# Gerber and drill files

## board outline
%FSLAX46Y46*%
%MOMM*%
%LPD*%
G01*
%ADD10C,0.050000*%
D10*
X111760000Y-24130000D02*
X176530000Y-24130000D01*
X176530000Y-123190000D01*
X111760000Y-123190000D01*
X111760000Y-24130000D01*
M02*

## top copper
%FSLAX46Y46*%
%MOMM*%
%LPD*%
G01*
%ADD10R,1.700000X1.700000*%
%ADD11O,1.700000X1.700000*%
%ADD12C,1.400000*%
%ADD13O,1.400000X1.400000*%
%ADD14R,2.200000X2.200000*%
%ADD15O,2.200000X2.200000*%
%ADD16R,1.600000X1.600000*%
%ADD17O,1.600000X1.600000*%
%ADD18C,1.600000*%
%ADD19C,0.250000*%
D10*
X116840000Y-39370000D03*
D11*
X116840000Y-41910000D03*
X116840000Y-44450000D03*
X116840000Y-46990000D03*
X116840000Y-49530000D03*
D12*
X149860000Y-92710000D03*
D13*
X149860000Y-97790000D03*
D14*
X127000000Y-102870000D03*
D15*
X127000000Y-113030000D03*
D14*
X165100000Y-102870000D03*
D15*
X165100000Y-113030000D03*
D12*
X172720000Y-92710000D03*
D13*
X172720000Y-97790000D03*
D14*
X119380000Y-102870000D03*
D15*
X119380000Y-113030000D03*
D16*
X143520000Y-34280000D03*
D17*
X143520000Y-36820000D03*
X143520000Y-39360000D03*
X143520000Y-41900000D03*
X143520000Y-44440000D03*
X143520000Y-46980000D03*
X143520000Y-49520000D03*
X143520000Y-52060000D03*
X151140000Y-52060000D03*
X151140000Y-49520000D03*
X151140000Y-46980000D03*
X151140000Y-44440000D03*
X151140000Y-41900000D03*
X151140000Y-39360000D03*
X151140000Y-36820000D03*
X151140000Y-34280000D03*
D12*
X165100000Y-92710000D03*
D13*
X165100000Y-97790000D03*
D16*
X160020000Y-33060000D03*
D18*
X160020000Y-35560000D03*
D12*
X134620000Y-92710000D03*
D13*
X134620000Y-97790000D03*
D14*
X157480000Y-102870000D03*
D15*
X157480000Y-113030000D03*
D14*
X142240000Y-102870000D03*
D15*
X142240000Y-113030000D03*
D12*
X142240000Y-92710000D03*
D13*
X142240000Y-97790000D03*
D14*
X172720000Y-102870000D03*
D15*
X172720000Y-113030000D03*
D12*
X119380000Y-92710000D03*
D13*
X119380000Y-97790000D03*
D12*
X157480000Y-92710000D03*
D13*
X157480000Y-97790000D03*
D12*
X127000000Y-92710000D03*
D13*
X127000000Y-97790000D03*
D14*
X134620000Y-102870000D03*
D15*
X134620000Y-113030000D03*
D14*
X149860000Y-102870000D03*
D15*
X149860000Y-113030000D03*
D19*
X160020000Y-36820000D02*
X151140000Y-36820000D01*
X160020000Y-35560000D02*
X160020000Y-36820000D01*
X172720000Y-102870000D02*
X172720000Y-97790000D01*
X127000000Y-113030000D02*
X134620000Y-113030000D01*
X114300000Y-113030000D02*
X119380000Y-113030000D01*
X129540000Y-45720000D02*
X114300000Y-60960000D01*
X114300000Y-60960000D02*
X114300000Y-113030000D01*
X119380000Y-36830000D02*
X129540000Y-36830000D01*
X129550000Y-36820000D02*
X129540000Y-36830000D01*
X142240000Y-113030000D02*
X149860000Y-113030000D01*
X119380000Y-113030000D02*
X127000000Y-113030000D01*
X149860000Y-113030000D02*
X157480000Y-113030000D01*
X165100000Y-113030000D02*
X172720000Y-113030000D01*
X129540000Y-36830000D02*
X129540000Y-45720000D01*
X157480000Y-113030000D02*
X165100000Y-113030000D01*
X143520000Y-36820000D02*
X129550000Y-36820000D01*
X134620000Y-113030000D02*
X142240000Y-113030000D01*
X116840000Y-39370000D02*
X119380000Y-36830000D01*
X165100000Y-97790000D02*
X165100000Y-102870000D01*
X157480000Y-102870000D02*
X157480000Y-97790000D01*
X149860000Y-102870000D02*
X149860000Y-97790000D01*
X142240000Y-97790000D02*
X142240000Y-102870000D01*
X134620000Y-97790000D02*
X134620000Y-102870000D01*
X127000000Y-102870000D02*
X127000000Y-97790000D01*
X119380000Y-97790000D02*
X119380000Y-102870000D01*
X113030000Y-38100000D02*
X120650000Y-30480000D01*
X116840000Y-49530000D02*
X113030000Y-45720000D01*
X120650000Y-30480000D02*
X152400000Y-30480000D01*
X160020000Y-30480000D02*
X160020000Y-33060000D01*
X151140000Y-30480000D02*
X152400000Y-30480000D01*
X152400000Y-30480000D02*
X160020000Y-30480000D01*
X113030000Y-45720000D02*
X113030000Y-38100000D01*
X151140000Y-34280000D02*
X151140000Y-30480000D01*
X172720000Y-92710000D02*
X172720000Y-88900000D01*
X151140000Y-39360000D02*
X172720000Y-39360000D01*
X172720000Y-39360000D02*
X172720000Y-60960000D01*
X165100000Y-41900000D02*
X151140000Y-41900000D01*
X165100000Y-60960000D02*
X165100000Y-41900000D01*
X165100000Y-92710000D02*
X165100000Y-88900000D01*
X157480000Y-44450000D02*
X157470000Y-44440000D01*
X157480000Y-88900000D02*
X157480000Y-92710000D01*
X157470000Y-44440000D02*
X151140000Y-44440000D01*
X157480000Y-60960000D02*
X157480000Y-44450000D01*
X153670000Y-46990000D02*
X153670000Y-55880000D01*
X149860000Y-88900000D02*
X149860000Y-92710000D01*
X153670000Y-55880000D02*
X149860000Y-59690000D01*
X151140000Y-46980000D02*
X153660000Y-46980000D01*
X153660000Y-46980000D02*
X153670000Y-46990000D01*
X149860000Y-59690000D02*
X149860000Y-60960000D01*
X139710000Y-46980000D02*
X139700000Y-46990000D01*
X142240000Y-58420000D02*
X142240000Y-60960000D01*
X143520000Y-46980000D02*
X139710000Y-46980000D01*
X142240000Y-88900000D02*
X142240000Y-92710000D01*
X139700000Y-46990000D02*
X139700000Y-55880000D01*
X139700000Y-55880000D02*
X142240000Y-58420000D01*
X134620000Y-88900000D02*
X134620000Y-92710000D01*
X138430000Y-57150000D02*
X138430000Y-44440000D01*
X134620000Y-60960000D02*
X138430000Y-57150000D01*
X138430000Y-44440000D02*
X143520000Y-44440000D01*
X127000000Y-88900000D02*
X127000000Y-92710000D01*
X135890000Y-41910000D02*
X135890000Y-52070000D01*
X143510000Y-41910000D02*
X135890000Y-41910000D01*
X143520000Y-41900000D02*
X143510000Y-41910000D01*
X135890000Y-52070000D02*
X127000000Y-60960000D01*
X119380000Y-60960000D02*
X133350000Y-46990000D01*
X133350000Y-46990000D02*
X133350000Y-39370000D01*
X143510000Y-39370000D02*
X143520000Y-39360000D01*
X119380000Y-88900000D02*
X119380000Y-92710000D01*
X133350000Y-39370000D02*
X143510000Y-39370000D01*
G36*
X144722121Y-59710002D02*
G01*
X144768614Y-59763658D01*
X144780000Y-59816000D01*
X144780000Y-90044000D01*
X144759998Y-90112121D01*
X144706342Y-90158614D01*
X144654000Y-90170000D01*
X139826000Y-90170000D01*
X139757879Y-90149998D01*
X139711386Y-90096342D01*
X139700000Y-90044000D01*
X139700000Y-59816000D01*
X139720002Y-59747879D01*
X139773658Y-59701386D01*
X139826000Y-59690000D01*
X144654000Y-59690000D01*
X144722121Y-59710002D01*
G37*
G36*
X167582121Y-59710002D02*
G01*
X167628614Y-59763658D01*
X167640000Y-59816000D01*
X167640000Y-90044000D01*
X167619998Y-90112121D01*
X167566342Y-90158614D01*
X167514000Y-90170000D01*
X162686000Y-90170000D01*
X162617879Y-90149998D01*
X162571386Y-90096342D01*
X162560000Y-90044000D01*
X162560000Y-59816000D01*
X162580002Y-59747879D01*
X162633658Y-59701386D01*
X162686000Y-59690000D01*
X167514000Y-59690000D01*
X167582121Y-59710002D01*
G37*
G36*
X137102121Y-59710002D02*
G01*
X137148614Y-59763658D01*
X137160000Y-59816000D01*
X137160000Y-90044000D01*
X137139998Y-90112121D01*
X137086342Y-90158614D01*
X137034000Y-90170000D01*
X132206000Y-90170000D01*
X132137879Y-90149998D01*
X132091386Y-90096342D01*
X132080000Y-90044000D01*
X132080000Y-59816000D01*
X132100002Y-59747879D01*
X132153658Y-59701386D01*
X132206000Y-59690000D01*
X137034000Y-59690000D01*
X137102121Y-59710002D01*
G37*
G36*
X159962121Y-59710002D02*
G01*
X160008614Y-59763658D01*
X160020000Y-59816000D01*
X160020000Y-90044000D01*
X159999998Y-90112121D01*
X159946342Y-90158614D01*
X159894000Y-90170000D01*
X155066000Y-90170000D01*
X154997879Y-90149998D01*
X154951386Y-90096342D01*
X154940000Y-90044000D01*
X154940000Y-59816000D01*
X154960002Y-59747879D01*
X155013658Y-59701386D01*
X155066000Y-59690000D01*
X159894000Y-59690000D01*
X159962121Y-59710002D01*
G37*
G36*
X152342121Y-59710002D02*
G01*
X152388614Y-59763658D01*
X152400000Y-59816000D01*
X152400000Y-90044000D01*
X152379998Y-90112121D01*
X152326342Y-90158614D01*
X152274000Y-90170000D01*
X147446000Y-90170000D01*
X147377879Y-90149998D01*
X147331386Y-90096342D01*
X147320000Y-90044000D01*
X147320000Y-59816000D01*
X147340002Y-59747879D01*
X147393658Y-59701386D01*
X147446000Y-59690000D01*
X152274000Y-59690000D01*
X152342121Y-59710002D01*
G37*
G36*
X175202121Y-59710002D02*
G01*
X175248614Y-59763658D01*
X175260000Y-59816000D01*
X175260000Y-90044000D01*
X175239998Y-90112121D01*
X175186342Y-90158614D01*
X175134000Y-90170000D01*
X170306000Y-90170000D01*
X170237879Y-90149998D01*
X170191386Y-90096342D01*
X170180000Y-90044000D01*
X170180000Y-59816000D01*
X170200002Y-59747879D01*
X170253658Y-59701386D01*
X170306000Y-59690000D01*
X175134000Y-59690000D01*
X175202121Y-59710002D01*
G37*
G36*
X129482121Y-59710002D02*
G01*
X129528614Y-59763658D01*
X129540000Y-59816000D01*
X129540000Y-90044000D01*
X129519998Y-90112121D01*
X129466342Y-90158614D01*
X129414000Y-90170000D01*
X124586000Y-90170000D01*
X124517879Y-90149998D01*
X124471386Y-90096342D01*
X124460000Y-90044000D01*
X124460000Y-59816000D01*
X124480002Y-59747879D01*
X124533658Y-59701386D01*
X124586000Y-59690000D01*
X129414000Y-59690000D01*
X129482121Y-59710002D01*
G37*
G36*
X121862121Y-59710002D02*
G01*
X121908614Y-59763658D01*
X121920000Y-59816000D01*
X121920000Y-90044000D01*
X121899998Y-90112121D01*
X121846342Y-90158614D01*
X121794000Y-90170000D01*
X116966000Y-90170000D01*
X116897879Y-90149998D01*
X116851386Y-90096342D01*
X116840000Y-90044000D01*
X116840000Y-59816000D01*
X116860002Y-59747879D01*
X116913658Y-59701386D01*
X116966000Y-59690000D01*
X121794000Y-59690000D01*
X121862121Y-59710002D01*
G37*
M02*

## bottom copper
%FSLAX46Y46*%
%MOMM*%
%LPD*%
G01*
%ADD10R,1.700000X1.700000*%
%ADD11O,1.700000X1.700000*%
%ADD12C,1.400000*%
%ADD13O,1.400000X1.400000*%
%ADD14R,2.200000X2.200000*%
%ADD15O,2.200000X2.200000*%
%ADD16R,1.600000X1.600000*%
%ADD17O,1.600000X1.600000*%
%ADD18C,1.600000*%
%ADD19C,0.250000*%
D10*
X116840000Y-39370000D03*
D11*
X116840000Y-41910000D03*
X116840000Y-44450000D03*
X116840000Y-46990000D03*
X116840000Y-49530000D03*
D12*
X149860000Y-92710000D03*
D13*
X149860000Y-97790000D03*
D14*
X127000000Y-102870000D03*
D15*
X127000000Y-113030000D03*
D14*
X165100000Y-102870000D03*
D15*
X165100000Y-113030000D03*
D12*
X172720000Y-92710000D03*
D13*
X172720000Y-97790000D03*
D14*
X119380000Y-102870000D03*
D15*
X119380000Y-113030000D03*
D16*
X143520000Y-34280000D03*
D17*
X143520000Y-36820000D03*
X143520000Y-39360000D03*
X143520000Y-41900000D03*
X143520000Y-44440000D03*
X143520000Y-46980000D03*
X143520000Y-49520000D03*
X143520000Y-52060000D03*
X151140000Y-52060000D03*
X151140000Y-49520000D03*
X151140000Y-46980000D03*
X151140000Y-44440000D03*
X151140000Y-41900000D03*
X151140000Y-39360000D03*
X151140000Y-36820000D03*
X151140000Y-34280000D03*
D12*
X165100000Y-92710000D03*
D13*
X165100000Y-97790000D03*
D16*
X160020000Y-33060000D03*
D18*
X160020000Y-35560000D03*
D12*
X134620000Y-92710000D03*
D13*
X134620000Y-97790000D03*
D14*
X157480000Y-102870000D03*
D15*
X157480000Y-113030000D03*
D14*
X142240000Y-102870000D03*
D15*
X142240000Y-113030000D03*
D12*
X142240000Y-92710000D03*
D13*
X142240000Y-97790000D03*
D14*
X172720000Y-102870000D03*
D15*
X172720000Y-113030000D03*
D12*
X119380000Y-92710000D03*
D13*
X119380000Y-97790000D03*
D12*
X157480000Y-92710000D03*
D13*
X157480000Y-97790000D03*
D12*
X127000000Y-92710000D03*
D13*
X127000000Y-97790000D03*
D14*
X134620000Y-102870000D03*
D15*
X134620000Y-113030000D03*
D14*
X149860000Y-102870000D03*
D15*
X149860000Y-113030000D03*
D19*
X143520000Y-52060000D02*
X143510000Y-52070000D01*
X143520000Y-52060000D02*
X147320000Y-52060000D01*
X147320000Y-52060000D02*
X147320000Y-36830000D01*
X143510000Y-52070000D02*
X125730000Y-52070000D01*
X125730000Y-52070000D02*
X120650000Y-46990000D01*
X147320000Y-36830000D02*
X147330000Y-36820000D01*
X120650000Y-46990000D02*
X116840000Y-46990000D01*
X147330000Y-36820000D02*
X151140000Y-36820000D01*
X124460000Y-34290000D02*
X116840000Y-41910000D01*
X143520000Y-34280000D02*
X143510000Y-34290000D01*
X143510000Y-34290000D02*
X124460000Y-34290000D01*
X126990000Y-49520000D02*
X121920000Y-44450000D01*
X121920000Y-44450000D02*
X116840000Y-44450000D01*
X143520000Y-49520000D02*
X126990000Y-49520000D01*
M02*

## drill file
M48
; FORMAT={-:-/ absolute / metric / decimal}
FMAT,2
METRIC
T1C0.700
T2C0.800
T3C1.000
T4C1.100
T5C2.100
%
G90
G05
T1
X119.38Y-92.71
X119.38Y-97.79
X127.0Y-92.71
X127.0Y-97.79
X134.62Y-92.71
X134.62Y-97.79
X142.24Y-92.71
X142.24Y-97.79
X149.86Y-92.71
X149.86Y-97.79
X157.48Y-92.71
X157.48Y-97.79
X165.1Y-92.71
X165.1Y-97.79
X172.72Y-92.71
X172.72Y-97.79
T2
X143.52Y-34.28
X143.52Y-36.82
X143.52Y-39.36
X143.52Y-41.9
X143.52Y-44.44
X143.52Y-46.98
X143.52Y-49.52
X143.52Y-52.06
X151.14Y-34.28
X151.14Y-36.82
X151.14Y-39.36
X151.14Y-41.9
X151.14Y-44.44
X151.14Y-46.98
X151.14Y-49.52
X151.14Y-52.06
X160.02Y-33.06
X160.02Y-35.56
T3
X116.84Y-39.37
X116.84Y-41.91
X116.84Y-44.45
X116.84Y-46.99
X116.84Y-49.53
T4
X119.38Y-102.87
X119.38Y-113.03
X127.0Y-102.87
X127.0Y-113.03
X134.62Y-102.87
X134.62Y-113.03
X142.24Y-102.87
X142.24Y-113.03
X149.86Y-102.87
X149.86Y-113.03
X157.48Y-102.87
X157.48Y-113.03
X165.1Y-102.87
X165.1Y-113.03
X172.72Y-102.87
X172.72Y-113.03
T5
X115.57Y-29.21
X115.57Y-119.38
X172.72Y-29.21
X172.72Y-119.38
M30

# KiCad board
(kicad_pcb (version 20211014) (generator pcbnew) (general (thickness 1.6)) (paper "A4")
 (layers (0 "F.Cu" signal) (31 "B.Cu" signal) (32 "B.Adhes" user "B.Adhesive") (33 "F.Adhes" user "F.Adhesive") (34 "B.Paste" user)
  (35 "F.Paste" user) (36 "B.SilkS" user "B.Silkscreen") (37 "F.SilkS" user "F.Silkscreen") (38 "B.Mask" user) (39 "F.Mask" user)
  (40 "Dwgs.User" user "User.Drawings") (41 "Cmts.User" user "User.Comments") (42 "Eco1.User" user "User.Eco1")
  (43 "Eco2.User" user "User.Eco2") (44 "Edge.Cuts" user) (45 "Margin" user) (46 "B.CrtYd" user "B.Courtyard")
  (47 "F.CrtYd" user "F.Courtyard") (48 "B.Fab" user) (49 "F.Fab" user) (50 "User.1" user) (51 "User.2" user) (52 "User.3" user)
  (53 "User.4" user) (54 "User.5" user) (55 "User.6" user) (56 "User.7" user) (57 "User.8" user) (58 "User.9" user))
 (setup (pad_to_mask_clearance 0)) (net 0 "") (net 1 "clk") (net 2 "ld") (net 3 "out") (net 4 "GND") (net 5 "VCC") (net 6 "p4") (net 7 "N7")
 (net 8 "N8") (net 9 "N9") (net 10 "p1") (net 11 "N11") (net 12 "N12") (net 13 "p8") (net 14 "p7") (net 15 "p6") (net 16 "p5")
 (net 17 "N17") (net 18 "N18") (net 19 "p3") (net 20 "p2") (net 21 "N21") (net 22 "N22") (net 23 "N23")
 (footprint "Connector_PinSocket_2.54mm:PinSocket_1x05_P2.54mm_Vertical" (layer "F.Cu") (at 116.84 39.37)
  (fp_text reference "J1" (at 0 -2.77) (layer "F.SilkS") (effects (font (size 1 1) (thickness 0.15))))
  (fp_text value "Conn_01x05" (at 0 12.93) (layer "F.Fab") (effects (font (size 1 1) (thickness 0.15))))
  (pad "1" thru_hole rect (at 0 0) (size 1.7 1.7) (drill 1) (layers *.Cu *.Mask) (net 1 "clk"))
  (pad "2" thru_hole oval (at 0 2.54) (size 1.7 1.7) (drill 1) (layers *.Cu *.Mask) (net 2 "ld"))
  (pad "3" thru_hole oval (at 0 5.08) (size 1.7 1.7) (drill 1) (layers *.Cu *.Mask) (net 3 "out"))
  (pad "4" thru_hole oval (at 0 7.62) (size 1.7 1.7) (drill 1) (layers *.Cu *.Mask) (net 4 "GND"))
  (pad "5" thru_hole oval (at 0 10.16) (size 1.7 1.7) (drill 1) (layers *.Cu *.Mask) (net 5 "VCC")))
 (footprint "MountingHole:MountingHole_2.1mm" (layer "F.Cu") (at 172.72 29.21)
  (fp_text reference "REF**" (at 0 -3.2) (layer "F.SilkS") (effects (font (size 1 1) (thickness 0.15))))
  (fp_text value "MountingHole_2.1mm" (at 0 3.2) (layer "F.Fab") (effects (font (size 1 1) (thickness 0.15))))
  (pad "" np_thru_hole circle (at 0 0) (size 2.1 2.1) (drill 2.1) (layers *.Cu *.Mask)))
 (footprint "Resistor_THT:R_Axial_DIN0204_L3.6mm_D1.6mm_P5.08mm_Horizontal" (layer "F.Cu") (at 149.86 92.71 -90)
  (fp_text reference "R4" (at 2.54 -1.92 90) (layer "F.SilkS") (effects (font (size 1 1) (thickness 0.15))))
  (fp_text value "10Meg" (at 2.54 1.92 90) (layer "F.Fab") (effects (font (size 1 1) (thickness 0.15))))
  (pad "1" thru_hole circle (at 0 0 270) (size 1.4 1.4) (drill 0.7) (layers *.Cu *.Mask) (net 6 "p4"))
  (pad "2" thru_hole oval (at 5.08 0 270) (size 1.4 1.4) (drill 0.7) (layers *.Cu *.Mask) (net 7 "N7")))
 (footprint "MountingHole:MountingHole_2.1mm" (layer "F.Cu") (at 115.57 119.38)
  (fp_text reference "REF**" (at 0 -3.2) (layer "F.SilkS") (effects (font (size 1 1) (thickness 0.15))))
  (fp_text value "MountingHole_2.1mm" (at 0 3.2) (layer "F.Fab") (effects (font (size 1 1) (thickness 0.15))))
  (pad "" np_thru_hole circle (at 0 0) (size 2.1 2.1) (drill 2.1) (layers *.Cu *.Mask)))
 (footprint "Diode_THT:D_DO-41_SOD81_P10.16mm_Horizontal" (layer "F.Cu") (at 127 102.87 -90)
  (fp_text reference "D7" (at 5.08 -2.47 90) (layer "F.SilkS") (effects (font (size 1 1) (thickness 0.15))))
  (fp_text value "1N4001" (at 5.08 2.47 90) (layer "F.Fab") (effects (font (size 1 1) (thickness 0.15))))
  (pad "1" thru_hole rect (at 0 0 270) (size 2.2 2.2) (drill 1.1) (layers *.Cu *.Mask) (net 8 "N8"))
  (pad "2" thru_hole oval (at 10.16 0 270) (size 2.2 2.2) (drill 1.1) (layers *.Cu *.Mask) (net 1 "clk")))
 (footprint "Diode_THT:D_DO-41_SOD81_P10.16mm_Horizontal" (layer "F.Cu") (at 165.1 102.87 -90)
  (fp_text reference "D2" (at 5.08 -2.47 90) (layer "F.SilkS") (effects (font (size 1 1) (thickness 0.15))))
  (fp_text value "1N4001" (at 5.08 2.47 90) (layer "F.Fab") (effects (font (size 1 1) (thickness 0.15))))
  (pad "1" thru_hole rect (at 0 0 270) (size 2.2 2.2) (drill 1.1) (layers *.Cu *.Mask) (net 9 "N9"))
  (pad "2" thru_hole oval (at 10.16 0 270) (size 2.2 2.2) (drill 1.1) (layers *.Cu *.Mask) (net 1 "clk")))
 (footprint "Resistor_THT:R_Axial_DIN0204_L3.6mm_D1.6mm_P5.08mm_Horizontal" (layer "F.Cu") (at 172.72 92.71 -90)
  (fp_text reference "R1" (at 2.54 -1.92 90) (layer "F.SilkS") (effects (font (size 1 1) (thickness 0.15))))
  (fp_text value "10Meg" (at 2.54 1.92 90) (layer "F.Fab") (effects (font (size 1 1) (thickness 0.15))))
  (pad "1" thru_hole circle (at 0 0 270) (size 1.4 1.4) (drill 0.7) (layers *.Cu *.Mask) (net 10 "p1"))
  (pad "2" thru_hole oval (at 5.08 0 270) (size 1.4 1.4) (drill 0.7) (layers *.Cu *.Mask) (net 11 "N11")))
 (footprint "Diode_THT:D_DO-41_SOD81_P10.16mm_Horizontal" (layer "F.Cu") (at 119.38 102.87 -90)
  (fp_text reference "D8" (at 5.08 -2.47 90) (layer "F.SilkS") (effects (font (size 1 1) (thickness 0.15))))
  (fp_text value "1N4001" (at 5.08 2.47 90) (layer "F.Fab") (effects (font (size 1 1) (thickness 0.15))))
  (pad "1" thru_hole rect (at 0 0 270) (size 2.2 2.2) (drill 1.1) (layers *.Cu *.Mask) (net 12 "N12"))
  (pad "2" thru_hole oval (at 10.16 0 270) (size 2.2 2.2) (drill 1.1) (layers *.Cu *.Mask) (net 1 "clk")))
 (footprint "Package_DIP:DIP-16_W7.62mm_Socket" (layer "F.Cu") (at 143.52 34.28)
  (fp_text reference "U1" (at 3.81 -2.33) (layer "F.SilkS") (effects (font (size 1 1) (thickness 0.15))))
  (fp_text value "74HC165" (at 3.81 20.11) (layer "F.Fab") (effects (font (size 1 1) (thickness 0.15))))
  (pad "1" thru_hole rect (at 0 0) (size 1.6 1.6) (drill 0.8) (layers *.Cu *.Mask) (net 2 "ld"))
  (pad "2" thru_hole oval (at 0 2.54) (size 1.6 1.6) (drill 0.8) (layers *.Cu *.Mask) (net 1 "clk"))
  (pad "3" thru_hole oval (at 0 5.08) (size 1.6 1.6) (drill 0.8) (layers *.Cu *.Mask) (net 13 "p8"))
  (pad "4" thru_hole oval (at 0 7.62) (size 1.6 1.6) (drill 0.8) (layers *.Cu *.Mask) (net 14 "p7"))
  (pad "5" thru_hole oval (at 0 10.16) (size 1.6 1.6) (drill 0.8) (layers *.Cu *.Mask) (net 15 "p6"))
  (pad "6" thru_hole oval (at 0 12.7) (size 1.6 1.6) (drill 0.8) (layers *.Cu *.Mask) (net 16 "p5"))
  (pad "7" thru_hole oval (at 0 15.24) (size 1.6 1.6) (drill 0.8) (layers *.Cu *.Mask) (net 3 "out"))
  (pad "8" thru_hole oval (at 0 17.78) (size 1.6 1.6) (drill 0.8) (layers *.Cu *.Mask) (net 4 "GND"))
  (pad "9" thru_hole oval (at 7.62 17.78) (size 1.6 1.6) (drill 0.8) (layers *.Cu *.Mask) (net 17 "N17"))
  (pad "10" thru_hole oval (at 7.62 15.24) (size 1.6 1.6) (drill 0.8) (layers *.Cu *.Mask) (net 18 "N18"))
  (pad "11" thru_hole oval (at 7.62 12.7) (size 1.6 1.6) (drill 0.8) (layers *.Cu *.Mask) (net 6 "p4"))
  (pad "12" thru_hole oval (at 7.62 10.16) (size 1.6 1.6) (drill 0.8) (layers *.Cu *.Mask) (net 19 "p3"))
  (pad "13" thru_hole oval (at 7.62 7.62) (size 1.6 1.6) (drill 0.8) (layers *.Cu *.Mask) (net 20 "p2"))
  (pad "14" thru_hole oval (at 7.62 5.08) (size 1.6 1.6) (drill 0.8) (layers *.Cu *.Mask) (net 10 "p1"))
  (pad "15" thru_hole oval (at 7.62 2.54) (size 1.6 1.6) (drill 0.8) (layers *.Cu *.Mask) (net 4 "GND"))
  (pad "16" thru_hole oval (at 7.62 0) (size 1.6 1.6) (drill 0.8) (layers *.Cu *.Mask) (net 5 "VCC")))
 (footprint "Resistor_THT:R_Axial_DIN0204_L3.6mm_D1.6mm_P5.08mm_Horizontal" (layer "F.Cu") (at 165.1 92.71 -90)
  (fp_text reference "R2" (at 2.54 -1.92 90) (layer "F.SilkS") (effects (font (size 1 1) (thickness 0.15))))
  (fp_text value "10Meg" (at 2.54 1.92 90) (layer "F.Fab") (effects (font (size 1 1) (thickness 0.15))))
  (pad "1" thru_hole circle (at 0 0 270) (size 1.4 1.4) (drill 0.7) (layers *.Cu *.Mask) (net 20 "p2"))
  (pad "2" thru_hole oval (at 5.08 0 270) (size 1.4 1.4) (drill 0.7) (layers *.Cu *.Mask) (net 9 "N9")))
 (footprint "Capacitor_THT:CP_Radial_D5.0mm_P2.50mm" (layer "F.Cu") (at 160.02 33.06 -90)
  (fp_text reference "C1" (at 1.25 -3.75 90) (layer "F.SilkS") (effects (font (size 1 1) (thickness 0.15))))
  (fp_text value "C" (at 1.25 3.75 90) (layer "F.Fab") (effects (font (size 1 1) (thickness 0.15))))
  (pad "1" thru_hole rect (at 0 0 270) (size 1.6 1.6) (drill 0.8) (layers *.Cu *.Mask) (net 5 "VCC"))
  (pad "2" thru_hole circle (at 2.5 0 270) (size 1.6 1.6) (drill 0.8) (layers *.Cu *.Mask) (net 4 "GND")))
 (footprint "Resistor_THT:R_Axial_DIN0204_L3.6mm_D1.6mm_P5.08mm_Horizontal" (layer "F.Cu") (at 134.62 92.71 -90)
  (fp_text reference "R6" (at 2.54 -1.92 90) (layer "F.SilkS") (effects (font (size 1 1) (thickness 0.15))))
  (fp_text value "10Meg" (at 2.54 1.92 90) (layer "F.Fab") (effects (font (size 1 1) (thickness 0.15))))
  (pad "1" thru_hole circle (at 0 0 270) (size 1.4 1.4) (drill 0.7) (layers *.Cu *.Mask) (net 15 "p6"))
  (pad "2" thru_hole oval (at 5.08 0 270) (size 1.4 1.4) (drill 0.7) (layers *.Cu *.Mask) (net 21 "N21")))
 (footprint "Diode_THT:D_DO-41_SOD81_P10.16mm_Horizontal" (layer "F.Cu") (at 157.48 102.87 -90)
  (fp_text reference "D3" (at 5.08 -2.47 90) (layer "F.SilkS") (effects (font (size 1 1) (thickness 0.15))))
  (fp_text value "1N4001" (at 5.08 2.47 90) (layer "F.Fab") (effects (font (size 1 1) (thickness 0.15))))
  (pad "1" thru_hole rect (at 0 0 270) (size 2.2 2.2) (drill 1.1) (layers *.Cu *.Mask) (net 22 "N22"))
  (pad "2" thru_hole oval (at 10.16 0 270) (size 2.2 2.2) (drill 1.1) (layers *.Cu *.Mask) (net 1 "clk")))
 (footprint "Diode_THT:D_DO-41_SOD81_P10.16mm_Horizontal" (layer "F.Cu") (at 142.24 102.87 -90)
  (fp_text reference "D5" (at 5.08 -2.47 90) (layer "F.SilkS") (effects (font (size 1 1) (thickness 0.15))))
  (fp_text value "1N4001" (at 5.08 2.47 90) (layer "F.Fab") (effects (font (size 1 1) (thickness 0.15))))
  (pad "1" thru_hole rect (at 0 0 270) (size 2.2 2.2) (drill 1.1) (layers *.Cu *.Mask) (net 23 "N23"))
  (pad "2" thru_hole oval (at 10.16 0 270) (size 2.2 2.2) (drill 1.1) (layers *.Cu *.Mask) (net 1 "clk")))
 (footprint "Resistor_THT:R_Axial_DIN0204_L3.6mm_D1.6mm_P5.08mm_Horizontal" (layer "F.Cu") (at 142.24 92.71 -90)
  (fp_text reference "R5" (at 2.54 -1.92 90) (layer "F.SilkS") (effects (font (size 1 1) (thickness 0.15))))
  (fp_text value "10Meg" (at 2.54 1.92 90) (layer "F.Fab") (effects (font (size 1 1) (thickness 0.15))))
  (pad "1" thru_hole circle (at 0 0 270) (size 1.4 1.4) (drill 0.7) (layers *.Cu *.Mask) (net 16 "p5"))
  (pad "2" thru_hole oval (at 5.08 0 270) (size 1.4 1.4) (drill 0.7) (layers *.Cu *.Mask) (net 23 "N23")))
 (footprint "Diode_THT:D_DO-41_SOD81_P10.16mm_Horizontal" (layer "F.Cu") (at 172.72 102.87 -90)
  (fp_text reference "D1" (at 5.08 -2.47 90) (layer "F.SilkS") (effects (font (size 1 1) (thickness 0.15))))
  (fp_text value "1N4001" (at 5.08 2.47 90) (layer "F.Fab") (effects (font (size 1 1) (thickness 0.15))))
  (pad "1" thru_hole rect (at 0 0 270) (size 2.2 2.2) (drill 1.1) (layers *.Cu *.Mask) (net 11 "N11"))
  (pad "2" thru_hole oval (at 10.16 0 270) (size 2.2 2.2) (drill 1.1) (layers *.Cu *.Mask) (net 1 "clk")))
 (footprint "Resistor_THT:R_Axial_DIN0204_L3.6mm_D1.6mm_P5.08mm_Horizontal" (layer "F.Cu") (at 119.38 92.71 -90)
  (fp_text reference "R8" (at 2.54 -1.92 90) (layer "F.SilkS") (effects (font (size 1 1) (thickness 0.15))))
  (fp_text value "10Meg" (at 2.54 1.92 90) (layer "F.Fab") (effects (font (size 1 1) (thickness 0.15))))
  (pad "1" thru_hole circle (at 0 0 270) (size 1.4 1.4) (drill 0.7) (layers *.Cu *.Mask) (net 13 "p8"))
  (pad "2" thru_hole oval (at 5.08 0 270) (size 1.4 1.4) (drill 0.7) (layers *.Cu *.Mask) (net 12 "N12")))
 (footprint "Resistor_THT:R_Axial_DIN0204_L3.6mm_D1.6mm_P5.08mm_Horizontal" (layer "F.Cu") (at 157.48 92.71 -90)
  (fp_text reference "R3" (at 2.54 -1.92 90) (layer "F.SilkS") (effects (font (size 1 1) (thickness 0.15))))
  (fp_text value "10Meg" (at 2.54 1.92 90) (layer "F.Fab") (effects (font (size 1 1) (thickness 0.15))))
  (pad "1" thru_hole circle (at 0 0 270) (size 1.4 1.4) (drill 0.7) (layers *.Cu *.Mask) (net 19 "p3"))
  (pad "2" thru_hole oval (at 5.08 0 270) (size 1.4 1.4) (drill 0.7) (layers *.Cu *.Mask) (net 22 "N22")))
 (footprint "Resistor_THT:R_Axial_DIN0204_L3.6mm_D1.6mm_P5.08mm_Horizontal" (layer "F.Cu") (at 127 92.71 -90)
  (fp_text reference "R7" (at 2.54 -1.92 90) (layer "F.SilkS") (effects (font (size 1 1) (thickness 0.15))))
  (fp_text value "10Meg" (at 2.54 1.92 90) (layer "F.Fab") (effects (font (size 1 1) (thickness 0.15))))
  (pad "1" thru_hole circle (at 0 0 270) (size 1.4 1.4) (drill 0.7) (layers *.Cu *.Mask) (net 14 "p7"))
  (pad "2" thru_hole oval (at 5.08 0 270) (size 1.4 1.4) (drill 0.7) (layers *.Cu *.Mask) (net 8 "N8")))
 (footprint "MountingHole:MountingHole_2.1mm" (layer "F.Cu") (at 172.72 119.38)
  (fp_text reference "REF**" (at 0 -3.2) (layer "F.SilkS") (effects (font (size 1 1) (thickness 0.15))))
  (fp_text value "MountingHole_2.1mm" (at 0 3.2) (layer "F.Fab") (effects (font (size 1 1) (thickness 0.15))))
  (pad "" np_thru_hole circle (at 0 0) (size 2.1 2.1) (drill 2.1) (layers *.Cu *.Mask)))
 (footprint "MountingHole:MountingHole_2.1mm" (layer "F.Cu") (at 115.57 29.21)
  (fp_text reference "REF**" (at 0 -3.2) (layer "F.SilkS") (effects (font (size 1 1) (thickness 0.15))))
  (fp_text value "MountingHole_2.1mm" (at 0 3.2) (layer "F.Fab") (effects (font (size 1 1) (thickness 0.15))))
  (pad "" np_thru_hole circle (at 0 0) (size 2.1 2.1) (drill 2.1) (layers *.Cu *.Mask)))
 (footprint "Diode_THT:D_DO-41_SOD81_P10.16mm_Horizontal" (layer "F.Cu") (at 134.62 102.87 -90)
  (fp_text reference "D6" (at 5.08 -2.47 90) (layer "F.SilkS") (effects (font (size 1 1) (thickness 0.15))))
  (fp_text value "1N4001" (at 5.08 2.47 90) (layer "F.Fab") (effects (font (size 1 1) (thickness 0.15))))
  (pad "1" thru_hole rect (at 0 0 270) (size 2.2 2.2) (drill 1.1) (layers *.Cu *.Mask) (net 21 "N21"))
  (pad "2" thru_hole oval (at 10.16 0 270) (size 2.2 2.2) (drill 1.1) (layers *.Cu *.Mask) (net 1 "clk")))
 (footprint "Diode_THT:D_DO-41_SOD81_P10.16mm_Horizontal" (layer "F.Cu") (at 149.86 102.87 -90)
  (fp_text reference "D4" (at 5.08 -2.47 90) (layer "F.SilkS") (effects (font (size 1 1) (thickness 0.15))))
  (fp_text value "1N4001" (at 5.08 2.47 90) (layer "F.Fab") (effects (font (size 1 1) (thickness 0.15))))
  (pad "1" thru_hole rect (at 0 0 270) (size 2.2 2.2) (drill 1.1) (layers *.Cu *.Mask) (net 7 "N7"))
  (pad "2" thru_hole oval (at 10.16 0 270) (size 2.2 2.2) (drill 1.1) (layers *.Cu *.Mask) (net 1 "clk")))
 (gr_rect (start 176.53 24.13) (end 111.76 123.19) (layer "Edge.Cuts") (width 0.05) (fill none))
 (segment (start 160.02 36.82) (end 151.14 36.82) (width 0.25) (layer "F.Cu") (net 4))
 (segment (start 160.02 35.56) (end 160.02 36.82) (width 0.25) (layer "F.Cu") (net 4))
 (segment (start 143.52 52.06) (end 143.51 52.07) (width 0.25) (layer "B.Cu") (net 4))
 (segment (start 143.52 52.06) (end 147.32 52.06) (width 0.25) (layer "B.Cu") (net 4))
 (segment (start 147.32 52.06) (end 147.32 36.83) (width 0.25) (layer "B.Cu") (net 4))
 (segment (start 143.51 52.07) (end 125.73 52.07) (width 0.25) (layer "B.Cu") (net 4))
 (segment (start 125.73 52.07) (end 120.65 46.99) (width 0.25) (layer "B.Cu") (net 4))
 (segment (start 147.32 36.83) (end 147.33 36.82) (width 0.25) (layer "B.Cu") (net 4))
 (segment (start 120.65 46.99) (end 116.84 46.99) (width 0.25) (layer "B.Cu") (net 4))
 (segment (start 147.33 36.82) (end 151.14 36.82) (width 0.25) (layer "B.Cu") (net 4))
 (segment (start 172.72 102.87) (end 172.72 97.79) (width 0.25) (layer "F.Cu") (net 11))
 (segment (start 127 113.03) (end 134.62 113.03) (width 0.25) (layer "F.Cu") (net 1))
 (segment (start 114.3 113.03) (end 119.38 113.03) (width 0.25) (layer "F.Cu") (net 1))
 (segment (start 129.54 45.72) (end 114.3 60.96) (width 0.25) (layer "F.Cu") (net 1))
 (segment (start 114.3 60.96) (end 114.3 113.03) (width 0.25) (layer "F.Cu") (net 1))
 (segment (start 119.38 36.83) (end 129.54 36.83) (width 0.25) (layer "F.Cu") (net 1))
 (segment (start 129.55 36.82) (end 129.54 36.83) (width 0.25) (layer "F.Cu") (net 1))
 (segment (start 142.24 113.03) (end 149.86 113.03) (width 0.25) (layer "F.Cu") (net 1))
 (segment (start 119.38 113.03) (end 127 113.03) (width 0.25) (layer "F.Cu") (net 1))
 (segment (start 149.86 113.03) (end 157.48 113.03) (width 0.25) (layer "F.Cu") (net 1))
 (segment (start 165.1 113.03) (end 172.72 113.03) (width 0.25) (layer "F.Cu") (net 1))
 (segment (start 129.54 36.83) (end 129.54 45.72) (width 0.25) (layer "F.Cu") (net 1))
 (segment (start 157.48 113.03) (end 165.1 113.03) (width 0.25) (layer "F.Cu") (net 1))
 (segment (start 143.52 36.82) (end 129.55 36.82) (width 0.25) (layer "F.Cu") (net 1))
 (segment (start 134.62 113.03) (end 142.24 113.03) (width 0.25) (layer "F.Cu") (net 1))
 (segment (start 116.84 39.37) (end 119.38 36.83) (width 0.25) (layer "F.Cu") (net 1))
 (segment (start 124.46 34.29) (end 116.84 41.91) (width 0.25) (layer "B.Cu") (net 2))
 (segment (start 143.52 34.28) (end 143.51 34.29) (width 0.25) (layer "B.Cu") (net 2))
 (segment (start 143.51 34.29) (end 124.46 34.29) (width 0.25) (layer "B.Cu") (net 2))
 (segment (start 165.1 97.79) (end 165.1 102.87) (width 0.25) (layer "F.Cu") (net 9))
 (segment (start 157.48 102.87) (end 157.48 97.79) (width 0.25) (layer "F.Cu") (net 22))
 (segment (start 149.86 102.87) (end 149.86 97.79) (width 0.25) (layer "F.Cu") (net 7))
 (segment (start 142.24 97.79) (end 142.24 102.87) (width 0.25) (layer "F.Cu") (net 23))
 (segment (start 134.62 97.79) (end 134.62 102.87) (width 0.25) (layer "F.Cu") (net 21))
 (segment (start 127 102.87) (end 127 97.79) (width 0.25) (layer "F.Cu") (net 8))
 (segment (start 119.38 97.79) (end 119.38 102.87) (width 0.25) (layer "F.Cu") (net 12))
 (segment (start 126.99 49.52) (end 121.92 44.45) (width 0.25) (layer "B.Cu") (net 3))
 (segment (start 121.92 44.45) (end 116.84 44.45) (width 0.25) (layer "B.Cu") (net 3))
 (segment (start 143.52 49.52) (end 126.99 49.52) (width 0.25) (layer "B.Cu") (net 3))
 (segment (start 113.03 38.1) (end 120.65 30.48) (width 0.25) (layer "F.Cu") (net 5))
 (segment (start 116.84 49.53) (end 113.03 45.72) (width 0.25) (layer "F.Cu") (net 5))
 (segment (start 120.65 30.48) (end 152.4 30.48) (width 0.25) (layer "F.Cu") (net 5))
 (segment (start 160.02 30.48) (end 160.02 33.06) (width 0.25) (layer "F.Cu") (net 5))
 (segment (start 151.14 30.48) (end 152.4 30.48) (width 0.25) (layer "F.Cu") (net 5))
 (segment (start 152.4 30.48) (end 160.02 30.48) (width 0.25) (layer "F.Cu") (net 5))
 (segment (start 113.03 45.72) (end 113.03 38.1) (width 0.25) (layer "F.Cu") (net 5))
 (segment (start 151.14 34.28) (end 151.14 30.48) (width 0.25) (layer "F.Cu") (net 5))
 (segment (start 172.72 92.71) (end 172.72 88.9) (width 0.25) (layer "F.Cu") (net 10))
 (segment (start 151.14 39.36) (end 172.72 39.36) (width 0.25) (layer "F.Cu") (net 10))
 (segment (start 172.72 39.36) (end 172.72 60.96) (width 0.25) (layer "F.Cu") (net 10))
 (segment (start 165.1 41.9) (end 151.14 41.9) (width 0.25) (layer "F.Cu") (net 20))
 (segment (start 165.1 60.96) (end 165.1 41.9) (width 0.25) (layer "F.Cu") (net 20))
 (segment (start 165.1 92.71) (end 165.1 88.9) (width 0.25) (layer "F.Cu") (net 20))
 (segment (start 157.48 44.45) (end 157.47 44.44) (width 0.25) (layer "F.Cu") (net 19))
 (segment (start 157.48 88.9) (end 157.48 92.71) (width 0.25) (layer "F.Cu") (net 19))
 (segment (start 157.47 44.44) (end 151.14 44.44) (width 0.25) (layer "F.Cu") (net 19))
 (segment (start 157.48 60.96) (end 157.48 44.45) (width 0.25) (layer "F.Cu") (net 19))
 (segment (start 153.67 46.99) (end 153.67 55.88) (width 0.25) (layer "F.Cu") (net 6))
 (segment (start 149.86 88.9) (end 149.86 92.71) (width 0.25) (layer "F.Cu") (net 6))
 (segment (start 153.67 55.88) (end 149.86 59.69) (width 0.25) (layer "F.Cu") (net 6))
 (segment (start 151.14 46.98) (end 153.66 46.98) (width 0.25) (layer "F.Cu") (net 6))
 (segment (start 153.66 46.98) (end 153.67 46.99) (width 0.25) (layer "F.Cu") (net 6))
 (segment (start 149.86 59.69) (end 149.86 60.96) (width 0.25) (layer "F.Cu") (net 6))
 (segment (start 139.71 46.98) (end 139.7 46.99) (width 0.25) (layer "F.Cu") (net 16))
 (segment (start 142.24 58.42) (end 142.24 60.96) (width 0.25) (layer "F.Cu") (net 16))
 (segment (start 143.52 46.98) (end 139.71 46.98) (width 0.25) (layer "F.Cu") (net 16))
 (segment (start 142.24 88.9) (end 142.24 92.71) (width 0.25) (layer "F.Cu") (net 16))
 (segment (start 139.7 46.99) (end 139.7 55.88) (width 0.25) (layer "F.Cu") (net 16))
 (segment (start 139.7 55.88) (end 142.24 58.42) (width 0.25) (layer "F.Cu") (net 16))
 (segment (start 134.62 88.9) (end 134.62 92.71) (width 0.25) (layer "F.Cu") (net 15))
 (segment (start 138.43 57.15) (end 138.43 44.44) (width 0.25) (layer "F.Cu") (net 15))
 (segment (start 134.62 60.96) (end 138.43 57.15) (width 0.25) (layer "F.Cu") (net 15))
 (segment (start 138.43 44.44) (end 143.52 44.44) (width 0.25) (layer "F.Cu") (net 15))
 (segment (start 127 88.9) (end 127 92.71) (width 0.25) (layer "F.Cu") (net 14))
 (segment (start 135.89 41.91) (end 135.89 52.07) (width 0.25) (layer "F.Cu") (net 14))
 (segment (start 143.51 41.91) (end 135.89 41.91) (width 0.25) (layer "F.Cu") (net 14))
 (segment (start 143.52 41.9) (end 143.51 41.91) (width 0.25) (layer "F.Cu") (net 14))
 (segment (start 135.89 52.07) (end 127 60.96) (width 0.25) (layer "F.Cu") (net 14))
 (segment (start 119.38 60.96) (end 133.35 46.99) (width 0.25) (layer "F.Cu") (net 13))
 (segment (start 133.35 46.99) (end 133.35 39.37) (width 0.25) (layer "F.Cu") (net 13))
 (segment (start 143.51 39.37) (end 143.52 39.36) (width 0.25) (layer "F.Cu") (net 13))
 (segment (start 119.38 88.9) (end 119.38 92.71) (width 0.25) (layer "F.Cu") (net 13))
 (segment (start 133.35 39.37) (end 143.51 39.37) (width 0.25) (layer "F.Cu") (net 13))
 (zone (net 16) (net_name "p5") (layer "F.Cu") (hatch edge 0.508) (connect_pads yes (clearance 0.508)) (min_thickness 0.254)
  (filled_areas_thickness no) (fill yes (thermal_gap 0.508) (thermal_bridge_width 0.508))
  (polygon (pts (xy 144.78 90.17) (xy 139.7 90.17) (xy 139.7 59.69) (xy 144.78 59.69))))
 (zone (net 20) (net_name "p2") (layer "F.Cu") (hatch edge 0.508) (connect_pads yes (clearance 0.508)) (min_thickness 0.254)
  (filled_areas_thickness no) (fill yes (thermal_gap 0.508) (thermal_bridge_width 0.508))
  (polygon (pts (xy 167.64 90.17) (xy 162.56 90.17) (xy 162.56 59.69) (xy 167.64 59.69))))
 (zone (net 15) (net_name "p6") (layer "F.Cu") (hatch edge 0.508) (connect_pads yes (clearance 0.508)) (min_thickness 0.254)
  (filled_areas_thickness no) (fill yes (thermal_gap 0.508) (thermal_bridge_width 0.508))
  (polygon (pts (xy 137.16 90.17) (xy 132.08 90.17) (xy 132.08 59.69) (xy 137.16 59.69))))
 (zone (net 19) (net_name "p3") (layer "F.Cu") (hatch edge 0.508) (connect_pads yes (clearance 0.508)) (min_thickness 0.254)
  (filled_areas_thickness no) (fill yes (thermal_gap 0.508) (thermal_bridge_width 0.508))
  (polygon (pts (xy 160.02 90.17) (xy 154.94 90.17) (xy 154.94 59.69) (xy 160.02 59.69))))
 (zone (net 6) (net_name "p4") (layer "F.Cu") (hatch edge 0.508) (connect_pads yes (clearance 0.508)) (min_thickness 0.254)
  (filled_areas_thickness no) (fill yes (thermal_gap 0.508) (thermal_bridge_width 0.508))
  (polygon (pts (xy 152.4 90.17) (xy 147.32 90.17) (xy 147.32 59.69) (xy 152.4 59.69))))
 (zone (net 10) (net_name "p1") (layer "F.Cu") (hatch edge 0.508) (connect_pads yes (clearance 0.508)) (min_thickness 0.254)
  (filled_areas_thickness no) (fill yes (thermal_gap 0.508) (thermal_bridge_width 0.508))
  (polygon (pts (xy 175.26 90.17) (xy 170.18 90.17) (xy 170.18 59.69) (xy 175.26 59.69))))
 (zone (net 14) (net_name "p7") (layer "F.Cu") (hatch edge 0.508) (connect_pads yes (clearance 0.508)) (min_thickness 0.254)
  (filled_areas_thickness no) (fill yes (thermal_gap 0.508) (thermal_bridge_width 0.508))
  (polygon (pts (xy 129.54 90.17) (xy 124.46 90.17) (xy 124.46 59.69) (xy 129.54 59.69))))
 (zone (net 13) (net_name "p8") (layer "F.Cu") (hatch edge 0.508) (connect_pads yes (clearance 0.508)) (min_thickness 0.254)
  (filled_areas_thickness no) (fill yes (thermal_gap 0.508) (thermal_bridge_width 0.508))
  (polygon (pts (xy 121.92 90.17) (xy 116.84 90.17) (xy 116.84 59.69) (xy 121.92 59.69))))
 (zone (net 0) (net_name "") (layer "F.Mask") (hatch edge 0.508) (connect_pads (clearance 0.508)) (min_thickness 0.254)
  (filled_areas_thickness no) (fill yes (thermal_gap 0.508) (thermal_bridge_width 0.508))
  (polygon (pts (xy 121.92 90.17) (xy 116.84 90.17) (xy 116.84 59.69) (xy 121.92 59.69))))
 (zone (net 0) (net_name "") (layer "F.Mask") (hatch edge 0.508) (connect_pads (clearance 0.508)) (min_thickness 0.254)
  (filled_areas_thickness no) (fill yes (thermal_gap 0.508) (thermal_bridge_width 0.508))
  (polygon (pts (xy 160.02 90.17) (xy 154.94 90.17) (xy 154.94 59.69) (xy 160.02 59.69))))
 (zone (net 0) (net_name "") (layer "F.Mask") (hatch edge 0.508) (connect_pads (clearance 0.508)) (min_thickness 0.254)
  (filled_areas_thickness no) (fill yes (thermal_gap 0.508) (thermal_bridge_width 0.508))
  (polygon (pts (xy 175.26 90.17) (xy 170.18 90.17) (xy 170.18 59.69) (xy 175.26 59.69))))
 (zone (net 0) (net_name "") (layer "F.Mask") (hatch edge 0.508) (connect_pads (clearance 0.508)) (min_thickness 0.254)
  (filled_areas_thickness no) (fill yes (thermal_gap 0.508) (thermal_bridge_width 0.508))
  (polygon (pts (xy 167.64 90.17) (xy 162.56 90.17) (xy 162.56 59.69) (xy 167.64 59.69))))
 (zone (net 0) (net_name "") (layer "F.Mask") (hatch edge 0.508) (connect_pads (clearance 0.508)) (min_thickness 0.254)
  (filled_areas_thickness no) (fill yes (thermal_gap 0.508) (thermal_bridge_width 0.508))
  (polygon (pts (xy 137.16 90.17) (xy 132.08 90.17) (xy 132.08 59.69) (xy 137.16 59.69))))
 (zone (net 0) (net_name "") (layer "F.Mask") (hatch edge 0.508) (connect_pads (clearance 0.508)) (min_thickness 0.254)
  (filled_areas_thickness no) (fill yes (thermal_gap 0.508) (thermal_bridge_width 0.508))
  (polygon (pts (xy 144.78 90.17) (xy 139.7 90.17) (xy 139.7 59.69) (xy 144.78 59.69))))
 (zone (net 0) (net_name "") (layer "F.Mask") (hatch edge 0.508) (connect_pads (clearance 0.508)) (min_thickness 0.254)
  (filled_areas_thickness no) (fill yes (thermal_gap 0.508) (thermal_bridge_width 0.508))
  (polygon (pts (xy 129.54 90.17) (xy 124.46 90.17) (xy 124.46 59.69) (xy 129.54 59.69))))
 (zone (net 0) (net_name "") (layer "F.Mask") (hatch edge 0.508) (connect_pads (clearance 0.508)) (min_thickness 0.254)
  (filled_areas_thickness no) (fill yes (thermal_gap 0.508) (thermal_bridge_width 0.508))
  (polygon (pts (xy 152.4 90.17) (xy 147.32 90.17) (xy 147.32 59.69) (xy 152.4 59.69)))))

